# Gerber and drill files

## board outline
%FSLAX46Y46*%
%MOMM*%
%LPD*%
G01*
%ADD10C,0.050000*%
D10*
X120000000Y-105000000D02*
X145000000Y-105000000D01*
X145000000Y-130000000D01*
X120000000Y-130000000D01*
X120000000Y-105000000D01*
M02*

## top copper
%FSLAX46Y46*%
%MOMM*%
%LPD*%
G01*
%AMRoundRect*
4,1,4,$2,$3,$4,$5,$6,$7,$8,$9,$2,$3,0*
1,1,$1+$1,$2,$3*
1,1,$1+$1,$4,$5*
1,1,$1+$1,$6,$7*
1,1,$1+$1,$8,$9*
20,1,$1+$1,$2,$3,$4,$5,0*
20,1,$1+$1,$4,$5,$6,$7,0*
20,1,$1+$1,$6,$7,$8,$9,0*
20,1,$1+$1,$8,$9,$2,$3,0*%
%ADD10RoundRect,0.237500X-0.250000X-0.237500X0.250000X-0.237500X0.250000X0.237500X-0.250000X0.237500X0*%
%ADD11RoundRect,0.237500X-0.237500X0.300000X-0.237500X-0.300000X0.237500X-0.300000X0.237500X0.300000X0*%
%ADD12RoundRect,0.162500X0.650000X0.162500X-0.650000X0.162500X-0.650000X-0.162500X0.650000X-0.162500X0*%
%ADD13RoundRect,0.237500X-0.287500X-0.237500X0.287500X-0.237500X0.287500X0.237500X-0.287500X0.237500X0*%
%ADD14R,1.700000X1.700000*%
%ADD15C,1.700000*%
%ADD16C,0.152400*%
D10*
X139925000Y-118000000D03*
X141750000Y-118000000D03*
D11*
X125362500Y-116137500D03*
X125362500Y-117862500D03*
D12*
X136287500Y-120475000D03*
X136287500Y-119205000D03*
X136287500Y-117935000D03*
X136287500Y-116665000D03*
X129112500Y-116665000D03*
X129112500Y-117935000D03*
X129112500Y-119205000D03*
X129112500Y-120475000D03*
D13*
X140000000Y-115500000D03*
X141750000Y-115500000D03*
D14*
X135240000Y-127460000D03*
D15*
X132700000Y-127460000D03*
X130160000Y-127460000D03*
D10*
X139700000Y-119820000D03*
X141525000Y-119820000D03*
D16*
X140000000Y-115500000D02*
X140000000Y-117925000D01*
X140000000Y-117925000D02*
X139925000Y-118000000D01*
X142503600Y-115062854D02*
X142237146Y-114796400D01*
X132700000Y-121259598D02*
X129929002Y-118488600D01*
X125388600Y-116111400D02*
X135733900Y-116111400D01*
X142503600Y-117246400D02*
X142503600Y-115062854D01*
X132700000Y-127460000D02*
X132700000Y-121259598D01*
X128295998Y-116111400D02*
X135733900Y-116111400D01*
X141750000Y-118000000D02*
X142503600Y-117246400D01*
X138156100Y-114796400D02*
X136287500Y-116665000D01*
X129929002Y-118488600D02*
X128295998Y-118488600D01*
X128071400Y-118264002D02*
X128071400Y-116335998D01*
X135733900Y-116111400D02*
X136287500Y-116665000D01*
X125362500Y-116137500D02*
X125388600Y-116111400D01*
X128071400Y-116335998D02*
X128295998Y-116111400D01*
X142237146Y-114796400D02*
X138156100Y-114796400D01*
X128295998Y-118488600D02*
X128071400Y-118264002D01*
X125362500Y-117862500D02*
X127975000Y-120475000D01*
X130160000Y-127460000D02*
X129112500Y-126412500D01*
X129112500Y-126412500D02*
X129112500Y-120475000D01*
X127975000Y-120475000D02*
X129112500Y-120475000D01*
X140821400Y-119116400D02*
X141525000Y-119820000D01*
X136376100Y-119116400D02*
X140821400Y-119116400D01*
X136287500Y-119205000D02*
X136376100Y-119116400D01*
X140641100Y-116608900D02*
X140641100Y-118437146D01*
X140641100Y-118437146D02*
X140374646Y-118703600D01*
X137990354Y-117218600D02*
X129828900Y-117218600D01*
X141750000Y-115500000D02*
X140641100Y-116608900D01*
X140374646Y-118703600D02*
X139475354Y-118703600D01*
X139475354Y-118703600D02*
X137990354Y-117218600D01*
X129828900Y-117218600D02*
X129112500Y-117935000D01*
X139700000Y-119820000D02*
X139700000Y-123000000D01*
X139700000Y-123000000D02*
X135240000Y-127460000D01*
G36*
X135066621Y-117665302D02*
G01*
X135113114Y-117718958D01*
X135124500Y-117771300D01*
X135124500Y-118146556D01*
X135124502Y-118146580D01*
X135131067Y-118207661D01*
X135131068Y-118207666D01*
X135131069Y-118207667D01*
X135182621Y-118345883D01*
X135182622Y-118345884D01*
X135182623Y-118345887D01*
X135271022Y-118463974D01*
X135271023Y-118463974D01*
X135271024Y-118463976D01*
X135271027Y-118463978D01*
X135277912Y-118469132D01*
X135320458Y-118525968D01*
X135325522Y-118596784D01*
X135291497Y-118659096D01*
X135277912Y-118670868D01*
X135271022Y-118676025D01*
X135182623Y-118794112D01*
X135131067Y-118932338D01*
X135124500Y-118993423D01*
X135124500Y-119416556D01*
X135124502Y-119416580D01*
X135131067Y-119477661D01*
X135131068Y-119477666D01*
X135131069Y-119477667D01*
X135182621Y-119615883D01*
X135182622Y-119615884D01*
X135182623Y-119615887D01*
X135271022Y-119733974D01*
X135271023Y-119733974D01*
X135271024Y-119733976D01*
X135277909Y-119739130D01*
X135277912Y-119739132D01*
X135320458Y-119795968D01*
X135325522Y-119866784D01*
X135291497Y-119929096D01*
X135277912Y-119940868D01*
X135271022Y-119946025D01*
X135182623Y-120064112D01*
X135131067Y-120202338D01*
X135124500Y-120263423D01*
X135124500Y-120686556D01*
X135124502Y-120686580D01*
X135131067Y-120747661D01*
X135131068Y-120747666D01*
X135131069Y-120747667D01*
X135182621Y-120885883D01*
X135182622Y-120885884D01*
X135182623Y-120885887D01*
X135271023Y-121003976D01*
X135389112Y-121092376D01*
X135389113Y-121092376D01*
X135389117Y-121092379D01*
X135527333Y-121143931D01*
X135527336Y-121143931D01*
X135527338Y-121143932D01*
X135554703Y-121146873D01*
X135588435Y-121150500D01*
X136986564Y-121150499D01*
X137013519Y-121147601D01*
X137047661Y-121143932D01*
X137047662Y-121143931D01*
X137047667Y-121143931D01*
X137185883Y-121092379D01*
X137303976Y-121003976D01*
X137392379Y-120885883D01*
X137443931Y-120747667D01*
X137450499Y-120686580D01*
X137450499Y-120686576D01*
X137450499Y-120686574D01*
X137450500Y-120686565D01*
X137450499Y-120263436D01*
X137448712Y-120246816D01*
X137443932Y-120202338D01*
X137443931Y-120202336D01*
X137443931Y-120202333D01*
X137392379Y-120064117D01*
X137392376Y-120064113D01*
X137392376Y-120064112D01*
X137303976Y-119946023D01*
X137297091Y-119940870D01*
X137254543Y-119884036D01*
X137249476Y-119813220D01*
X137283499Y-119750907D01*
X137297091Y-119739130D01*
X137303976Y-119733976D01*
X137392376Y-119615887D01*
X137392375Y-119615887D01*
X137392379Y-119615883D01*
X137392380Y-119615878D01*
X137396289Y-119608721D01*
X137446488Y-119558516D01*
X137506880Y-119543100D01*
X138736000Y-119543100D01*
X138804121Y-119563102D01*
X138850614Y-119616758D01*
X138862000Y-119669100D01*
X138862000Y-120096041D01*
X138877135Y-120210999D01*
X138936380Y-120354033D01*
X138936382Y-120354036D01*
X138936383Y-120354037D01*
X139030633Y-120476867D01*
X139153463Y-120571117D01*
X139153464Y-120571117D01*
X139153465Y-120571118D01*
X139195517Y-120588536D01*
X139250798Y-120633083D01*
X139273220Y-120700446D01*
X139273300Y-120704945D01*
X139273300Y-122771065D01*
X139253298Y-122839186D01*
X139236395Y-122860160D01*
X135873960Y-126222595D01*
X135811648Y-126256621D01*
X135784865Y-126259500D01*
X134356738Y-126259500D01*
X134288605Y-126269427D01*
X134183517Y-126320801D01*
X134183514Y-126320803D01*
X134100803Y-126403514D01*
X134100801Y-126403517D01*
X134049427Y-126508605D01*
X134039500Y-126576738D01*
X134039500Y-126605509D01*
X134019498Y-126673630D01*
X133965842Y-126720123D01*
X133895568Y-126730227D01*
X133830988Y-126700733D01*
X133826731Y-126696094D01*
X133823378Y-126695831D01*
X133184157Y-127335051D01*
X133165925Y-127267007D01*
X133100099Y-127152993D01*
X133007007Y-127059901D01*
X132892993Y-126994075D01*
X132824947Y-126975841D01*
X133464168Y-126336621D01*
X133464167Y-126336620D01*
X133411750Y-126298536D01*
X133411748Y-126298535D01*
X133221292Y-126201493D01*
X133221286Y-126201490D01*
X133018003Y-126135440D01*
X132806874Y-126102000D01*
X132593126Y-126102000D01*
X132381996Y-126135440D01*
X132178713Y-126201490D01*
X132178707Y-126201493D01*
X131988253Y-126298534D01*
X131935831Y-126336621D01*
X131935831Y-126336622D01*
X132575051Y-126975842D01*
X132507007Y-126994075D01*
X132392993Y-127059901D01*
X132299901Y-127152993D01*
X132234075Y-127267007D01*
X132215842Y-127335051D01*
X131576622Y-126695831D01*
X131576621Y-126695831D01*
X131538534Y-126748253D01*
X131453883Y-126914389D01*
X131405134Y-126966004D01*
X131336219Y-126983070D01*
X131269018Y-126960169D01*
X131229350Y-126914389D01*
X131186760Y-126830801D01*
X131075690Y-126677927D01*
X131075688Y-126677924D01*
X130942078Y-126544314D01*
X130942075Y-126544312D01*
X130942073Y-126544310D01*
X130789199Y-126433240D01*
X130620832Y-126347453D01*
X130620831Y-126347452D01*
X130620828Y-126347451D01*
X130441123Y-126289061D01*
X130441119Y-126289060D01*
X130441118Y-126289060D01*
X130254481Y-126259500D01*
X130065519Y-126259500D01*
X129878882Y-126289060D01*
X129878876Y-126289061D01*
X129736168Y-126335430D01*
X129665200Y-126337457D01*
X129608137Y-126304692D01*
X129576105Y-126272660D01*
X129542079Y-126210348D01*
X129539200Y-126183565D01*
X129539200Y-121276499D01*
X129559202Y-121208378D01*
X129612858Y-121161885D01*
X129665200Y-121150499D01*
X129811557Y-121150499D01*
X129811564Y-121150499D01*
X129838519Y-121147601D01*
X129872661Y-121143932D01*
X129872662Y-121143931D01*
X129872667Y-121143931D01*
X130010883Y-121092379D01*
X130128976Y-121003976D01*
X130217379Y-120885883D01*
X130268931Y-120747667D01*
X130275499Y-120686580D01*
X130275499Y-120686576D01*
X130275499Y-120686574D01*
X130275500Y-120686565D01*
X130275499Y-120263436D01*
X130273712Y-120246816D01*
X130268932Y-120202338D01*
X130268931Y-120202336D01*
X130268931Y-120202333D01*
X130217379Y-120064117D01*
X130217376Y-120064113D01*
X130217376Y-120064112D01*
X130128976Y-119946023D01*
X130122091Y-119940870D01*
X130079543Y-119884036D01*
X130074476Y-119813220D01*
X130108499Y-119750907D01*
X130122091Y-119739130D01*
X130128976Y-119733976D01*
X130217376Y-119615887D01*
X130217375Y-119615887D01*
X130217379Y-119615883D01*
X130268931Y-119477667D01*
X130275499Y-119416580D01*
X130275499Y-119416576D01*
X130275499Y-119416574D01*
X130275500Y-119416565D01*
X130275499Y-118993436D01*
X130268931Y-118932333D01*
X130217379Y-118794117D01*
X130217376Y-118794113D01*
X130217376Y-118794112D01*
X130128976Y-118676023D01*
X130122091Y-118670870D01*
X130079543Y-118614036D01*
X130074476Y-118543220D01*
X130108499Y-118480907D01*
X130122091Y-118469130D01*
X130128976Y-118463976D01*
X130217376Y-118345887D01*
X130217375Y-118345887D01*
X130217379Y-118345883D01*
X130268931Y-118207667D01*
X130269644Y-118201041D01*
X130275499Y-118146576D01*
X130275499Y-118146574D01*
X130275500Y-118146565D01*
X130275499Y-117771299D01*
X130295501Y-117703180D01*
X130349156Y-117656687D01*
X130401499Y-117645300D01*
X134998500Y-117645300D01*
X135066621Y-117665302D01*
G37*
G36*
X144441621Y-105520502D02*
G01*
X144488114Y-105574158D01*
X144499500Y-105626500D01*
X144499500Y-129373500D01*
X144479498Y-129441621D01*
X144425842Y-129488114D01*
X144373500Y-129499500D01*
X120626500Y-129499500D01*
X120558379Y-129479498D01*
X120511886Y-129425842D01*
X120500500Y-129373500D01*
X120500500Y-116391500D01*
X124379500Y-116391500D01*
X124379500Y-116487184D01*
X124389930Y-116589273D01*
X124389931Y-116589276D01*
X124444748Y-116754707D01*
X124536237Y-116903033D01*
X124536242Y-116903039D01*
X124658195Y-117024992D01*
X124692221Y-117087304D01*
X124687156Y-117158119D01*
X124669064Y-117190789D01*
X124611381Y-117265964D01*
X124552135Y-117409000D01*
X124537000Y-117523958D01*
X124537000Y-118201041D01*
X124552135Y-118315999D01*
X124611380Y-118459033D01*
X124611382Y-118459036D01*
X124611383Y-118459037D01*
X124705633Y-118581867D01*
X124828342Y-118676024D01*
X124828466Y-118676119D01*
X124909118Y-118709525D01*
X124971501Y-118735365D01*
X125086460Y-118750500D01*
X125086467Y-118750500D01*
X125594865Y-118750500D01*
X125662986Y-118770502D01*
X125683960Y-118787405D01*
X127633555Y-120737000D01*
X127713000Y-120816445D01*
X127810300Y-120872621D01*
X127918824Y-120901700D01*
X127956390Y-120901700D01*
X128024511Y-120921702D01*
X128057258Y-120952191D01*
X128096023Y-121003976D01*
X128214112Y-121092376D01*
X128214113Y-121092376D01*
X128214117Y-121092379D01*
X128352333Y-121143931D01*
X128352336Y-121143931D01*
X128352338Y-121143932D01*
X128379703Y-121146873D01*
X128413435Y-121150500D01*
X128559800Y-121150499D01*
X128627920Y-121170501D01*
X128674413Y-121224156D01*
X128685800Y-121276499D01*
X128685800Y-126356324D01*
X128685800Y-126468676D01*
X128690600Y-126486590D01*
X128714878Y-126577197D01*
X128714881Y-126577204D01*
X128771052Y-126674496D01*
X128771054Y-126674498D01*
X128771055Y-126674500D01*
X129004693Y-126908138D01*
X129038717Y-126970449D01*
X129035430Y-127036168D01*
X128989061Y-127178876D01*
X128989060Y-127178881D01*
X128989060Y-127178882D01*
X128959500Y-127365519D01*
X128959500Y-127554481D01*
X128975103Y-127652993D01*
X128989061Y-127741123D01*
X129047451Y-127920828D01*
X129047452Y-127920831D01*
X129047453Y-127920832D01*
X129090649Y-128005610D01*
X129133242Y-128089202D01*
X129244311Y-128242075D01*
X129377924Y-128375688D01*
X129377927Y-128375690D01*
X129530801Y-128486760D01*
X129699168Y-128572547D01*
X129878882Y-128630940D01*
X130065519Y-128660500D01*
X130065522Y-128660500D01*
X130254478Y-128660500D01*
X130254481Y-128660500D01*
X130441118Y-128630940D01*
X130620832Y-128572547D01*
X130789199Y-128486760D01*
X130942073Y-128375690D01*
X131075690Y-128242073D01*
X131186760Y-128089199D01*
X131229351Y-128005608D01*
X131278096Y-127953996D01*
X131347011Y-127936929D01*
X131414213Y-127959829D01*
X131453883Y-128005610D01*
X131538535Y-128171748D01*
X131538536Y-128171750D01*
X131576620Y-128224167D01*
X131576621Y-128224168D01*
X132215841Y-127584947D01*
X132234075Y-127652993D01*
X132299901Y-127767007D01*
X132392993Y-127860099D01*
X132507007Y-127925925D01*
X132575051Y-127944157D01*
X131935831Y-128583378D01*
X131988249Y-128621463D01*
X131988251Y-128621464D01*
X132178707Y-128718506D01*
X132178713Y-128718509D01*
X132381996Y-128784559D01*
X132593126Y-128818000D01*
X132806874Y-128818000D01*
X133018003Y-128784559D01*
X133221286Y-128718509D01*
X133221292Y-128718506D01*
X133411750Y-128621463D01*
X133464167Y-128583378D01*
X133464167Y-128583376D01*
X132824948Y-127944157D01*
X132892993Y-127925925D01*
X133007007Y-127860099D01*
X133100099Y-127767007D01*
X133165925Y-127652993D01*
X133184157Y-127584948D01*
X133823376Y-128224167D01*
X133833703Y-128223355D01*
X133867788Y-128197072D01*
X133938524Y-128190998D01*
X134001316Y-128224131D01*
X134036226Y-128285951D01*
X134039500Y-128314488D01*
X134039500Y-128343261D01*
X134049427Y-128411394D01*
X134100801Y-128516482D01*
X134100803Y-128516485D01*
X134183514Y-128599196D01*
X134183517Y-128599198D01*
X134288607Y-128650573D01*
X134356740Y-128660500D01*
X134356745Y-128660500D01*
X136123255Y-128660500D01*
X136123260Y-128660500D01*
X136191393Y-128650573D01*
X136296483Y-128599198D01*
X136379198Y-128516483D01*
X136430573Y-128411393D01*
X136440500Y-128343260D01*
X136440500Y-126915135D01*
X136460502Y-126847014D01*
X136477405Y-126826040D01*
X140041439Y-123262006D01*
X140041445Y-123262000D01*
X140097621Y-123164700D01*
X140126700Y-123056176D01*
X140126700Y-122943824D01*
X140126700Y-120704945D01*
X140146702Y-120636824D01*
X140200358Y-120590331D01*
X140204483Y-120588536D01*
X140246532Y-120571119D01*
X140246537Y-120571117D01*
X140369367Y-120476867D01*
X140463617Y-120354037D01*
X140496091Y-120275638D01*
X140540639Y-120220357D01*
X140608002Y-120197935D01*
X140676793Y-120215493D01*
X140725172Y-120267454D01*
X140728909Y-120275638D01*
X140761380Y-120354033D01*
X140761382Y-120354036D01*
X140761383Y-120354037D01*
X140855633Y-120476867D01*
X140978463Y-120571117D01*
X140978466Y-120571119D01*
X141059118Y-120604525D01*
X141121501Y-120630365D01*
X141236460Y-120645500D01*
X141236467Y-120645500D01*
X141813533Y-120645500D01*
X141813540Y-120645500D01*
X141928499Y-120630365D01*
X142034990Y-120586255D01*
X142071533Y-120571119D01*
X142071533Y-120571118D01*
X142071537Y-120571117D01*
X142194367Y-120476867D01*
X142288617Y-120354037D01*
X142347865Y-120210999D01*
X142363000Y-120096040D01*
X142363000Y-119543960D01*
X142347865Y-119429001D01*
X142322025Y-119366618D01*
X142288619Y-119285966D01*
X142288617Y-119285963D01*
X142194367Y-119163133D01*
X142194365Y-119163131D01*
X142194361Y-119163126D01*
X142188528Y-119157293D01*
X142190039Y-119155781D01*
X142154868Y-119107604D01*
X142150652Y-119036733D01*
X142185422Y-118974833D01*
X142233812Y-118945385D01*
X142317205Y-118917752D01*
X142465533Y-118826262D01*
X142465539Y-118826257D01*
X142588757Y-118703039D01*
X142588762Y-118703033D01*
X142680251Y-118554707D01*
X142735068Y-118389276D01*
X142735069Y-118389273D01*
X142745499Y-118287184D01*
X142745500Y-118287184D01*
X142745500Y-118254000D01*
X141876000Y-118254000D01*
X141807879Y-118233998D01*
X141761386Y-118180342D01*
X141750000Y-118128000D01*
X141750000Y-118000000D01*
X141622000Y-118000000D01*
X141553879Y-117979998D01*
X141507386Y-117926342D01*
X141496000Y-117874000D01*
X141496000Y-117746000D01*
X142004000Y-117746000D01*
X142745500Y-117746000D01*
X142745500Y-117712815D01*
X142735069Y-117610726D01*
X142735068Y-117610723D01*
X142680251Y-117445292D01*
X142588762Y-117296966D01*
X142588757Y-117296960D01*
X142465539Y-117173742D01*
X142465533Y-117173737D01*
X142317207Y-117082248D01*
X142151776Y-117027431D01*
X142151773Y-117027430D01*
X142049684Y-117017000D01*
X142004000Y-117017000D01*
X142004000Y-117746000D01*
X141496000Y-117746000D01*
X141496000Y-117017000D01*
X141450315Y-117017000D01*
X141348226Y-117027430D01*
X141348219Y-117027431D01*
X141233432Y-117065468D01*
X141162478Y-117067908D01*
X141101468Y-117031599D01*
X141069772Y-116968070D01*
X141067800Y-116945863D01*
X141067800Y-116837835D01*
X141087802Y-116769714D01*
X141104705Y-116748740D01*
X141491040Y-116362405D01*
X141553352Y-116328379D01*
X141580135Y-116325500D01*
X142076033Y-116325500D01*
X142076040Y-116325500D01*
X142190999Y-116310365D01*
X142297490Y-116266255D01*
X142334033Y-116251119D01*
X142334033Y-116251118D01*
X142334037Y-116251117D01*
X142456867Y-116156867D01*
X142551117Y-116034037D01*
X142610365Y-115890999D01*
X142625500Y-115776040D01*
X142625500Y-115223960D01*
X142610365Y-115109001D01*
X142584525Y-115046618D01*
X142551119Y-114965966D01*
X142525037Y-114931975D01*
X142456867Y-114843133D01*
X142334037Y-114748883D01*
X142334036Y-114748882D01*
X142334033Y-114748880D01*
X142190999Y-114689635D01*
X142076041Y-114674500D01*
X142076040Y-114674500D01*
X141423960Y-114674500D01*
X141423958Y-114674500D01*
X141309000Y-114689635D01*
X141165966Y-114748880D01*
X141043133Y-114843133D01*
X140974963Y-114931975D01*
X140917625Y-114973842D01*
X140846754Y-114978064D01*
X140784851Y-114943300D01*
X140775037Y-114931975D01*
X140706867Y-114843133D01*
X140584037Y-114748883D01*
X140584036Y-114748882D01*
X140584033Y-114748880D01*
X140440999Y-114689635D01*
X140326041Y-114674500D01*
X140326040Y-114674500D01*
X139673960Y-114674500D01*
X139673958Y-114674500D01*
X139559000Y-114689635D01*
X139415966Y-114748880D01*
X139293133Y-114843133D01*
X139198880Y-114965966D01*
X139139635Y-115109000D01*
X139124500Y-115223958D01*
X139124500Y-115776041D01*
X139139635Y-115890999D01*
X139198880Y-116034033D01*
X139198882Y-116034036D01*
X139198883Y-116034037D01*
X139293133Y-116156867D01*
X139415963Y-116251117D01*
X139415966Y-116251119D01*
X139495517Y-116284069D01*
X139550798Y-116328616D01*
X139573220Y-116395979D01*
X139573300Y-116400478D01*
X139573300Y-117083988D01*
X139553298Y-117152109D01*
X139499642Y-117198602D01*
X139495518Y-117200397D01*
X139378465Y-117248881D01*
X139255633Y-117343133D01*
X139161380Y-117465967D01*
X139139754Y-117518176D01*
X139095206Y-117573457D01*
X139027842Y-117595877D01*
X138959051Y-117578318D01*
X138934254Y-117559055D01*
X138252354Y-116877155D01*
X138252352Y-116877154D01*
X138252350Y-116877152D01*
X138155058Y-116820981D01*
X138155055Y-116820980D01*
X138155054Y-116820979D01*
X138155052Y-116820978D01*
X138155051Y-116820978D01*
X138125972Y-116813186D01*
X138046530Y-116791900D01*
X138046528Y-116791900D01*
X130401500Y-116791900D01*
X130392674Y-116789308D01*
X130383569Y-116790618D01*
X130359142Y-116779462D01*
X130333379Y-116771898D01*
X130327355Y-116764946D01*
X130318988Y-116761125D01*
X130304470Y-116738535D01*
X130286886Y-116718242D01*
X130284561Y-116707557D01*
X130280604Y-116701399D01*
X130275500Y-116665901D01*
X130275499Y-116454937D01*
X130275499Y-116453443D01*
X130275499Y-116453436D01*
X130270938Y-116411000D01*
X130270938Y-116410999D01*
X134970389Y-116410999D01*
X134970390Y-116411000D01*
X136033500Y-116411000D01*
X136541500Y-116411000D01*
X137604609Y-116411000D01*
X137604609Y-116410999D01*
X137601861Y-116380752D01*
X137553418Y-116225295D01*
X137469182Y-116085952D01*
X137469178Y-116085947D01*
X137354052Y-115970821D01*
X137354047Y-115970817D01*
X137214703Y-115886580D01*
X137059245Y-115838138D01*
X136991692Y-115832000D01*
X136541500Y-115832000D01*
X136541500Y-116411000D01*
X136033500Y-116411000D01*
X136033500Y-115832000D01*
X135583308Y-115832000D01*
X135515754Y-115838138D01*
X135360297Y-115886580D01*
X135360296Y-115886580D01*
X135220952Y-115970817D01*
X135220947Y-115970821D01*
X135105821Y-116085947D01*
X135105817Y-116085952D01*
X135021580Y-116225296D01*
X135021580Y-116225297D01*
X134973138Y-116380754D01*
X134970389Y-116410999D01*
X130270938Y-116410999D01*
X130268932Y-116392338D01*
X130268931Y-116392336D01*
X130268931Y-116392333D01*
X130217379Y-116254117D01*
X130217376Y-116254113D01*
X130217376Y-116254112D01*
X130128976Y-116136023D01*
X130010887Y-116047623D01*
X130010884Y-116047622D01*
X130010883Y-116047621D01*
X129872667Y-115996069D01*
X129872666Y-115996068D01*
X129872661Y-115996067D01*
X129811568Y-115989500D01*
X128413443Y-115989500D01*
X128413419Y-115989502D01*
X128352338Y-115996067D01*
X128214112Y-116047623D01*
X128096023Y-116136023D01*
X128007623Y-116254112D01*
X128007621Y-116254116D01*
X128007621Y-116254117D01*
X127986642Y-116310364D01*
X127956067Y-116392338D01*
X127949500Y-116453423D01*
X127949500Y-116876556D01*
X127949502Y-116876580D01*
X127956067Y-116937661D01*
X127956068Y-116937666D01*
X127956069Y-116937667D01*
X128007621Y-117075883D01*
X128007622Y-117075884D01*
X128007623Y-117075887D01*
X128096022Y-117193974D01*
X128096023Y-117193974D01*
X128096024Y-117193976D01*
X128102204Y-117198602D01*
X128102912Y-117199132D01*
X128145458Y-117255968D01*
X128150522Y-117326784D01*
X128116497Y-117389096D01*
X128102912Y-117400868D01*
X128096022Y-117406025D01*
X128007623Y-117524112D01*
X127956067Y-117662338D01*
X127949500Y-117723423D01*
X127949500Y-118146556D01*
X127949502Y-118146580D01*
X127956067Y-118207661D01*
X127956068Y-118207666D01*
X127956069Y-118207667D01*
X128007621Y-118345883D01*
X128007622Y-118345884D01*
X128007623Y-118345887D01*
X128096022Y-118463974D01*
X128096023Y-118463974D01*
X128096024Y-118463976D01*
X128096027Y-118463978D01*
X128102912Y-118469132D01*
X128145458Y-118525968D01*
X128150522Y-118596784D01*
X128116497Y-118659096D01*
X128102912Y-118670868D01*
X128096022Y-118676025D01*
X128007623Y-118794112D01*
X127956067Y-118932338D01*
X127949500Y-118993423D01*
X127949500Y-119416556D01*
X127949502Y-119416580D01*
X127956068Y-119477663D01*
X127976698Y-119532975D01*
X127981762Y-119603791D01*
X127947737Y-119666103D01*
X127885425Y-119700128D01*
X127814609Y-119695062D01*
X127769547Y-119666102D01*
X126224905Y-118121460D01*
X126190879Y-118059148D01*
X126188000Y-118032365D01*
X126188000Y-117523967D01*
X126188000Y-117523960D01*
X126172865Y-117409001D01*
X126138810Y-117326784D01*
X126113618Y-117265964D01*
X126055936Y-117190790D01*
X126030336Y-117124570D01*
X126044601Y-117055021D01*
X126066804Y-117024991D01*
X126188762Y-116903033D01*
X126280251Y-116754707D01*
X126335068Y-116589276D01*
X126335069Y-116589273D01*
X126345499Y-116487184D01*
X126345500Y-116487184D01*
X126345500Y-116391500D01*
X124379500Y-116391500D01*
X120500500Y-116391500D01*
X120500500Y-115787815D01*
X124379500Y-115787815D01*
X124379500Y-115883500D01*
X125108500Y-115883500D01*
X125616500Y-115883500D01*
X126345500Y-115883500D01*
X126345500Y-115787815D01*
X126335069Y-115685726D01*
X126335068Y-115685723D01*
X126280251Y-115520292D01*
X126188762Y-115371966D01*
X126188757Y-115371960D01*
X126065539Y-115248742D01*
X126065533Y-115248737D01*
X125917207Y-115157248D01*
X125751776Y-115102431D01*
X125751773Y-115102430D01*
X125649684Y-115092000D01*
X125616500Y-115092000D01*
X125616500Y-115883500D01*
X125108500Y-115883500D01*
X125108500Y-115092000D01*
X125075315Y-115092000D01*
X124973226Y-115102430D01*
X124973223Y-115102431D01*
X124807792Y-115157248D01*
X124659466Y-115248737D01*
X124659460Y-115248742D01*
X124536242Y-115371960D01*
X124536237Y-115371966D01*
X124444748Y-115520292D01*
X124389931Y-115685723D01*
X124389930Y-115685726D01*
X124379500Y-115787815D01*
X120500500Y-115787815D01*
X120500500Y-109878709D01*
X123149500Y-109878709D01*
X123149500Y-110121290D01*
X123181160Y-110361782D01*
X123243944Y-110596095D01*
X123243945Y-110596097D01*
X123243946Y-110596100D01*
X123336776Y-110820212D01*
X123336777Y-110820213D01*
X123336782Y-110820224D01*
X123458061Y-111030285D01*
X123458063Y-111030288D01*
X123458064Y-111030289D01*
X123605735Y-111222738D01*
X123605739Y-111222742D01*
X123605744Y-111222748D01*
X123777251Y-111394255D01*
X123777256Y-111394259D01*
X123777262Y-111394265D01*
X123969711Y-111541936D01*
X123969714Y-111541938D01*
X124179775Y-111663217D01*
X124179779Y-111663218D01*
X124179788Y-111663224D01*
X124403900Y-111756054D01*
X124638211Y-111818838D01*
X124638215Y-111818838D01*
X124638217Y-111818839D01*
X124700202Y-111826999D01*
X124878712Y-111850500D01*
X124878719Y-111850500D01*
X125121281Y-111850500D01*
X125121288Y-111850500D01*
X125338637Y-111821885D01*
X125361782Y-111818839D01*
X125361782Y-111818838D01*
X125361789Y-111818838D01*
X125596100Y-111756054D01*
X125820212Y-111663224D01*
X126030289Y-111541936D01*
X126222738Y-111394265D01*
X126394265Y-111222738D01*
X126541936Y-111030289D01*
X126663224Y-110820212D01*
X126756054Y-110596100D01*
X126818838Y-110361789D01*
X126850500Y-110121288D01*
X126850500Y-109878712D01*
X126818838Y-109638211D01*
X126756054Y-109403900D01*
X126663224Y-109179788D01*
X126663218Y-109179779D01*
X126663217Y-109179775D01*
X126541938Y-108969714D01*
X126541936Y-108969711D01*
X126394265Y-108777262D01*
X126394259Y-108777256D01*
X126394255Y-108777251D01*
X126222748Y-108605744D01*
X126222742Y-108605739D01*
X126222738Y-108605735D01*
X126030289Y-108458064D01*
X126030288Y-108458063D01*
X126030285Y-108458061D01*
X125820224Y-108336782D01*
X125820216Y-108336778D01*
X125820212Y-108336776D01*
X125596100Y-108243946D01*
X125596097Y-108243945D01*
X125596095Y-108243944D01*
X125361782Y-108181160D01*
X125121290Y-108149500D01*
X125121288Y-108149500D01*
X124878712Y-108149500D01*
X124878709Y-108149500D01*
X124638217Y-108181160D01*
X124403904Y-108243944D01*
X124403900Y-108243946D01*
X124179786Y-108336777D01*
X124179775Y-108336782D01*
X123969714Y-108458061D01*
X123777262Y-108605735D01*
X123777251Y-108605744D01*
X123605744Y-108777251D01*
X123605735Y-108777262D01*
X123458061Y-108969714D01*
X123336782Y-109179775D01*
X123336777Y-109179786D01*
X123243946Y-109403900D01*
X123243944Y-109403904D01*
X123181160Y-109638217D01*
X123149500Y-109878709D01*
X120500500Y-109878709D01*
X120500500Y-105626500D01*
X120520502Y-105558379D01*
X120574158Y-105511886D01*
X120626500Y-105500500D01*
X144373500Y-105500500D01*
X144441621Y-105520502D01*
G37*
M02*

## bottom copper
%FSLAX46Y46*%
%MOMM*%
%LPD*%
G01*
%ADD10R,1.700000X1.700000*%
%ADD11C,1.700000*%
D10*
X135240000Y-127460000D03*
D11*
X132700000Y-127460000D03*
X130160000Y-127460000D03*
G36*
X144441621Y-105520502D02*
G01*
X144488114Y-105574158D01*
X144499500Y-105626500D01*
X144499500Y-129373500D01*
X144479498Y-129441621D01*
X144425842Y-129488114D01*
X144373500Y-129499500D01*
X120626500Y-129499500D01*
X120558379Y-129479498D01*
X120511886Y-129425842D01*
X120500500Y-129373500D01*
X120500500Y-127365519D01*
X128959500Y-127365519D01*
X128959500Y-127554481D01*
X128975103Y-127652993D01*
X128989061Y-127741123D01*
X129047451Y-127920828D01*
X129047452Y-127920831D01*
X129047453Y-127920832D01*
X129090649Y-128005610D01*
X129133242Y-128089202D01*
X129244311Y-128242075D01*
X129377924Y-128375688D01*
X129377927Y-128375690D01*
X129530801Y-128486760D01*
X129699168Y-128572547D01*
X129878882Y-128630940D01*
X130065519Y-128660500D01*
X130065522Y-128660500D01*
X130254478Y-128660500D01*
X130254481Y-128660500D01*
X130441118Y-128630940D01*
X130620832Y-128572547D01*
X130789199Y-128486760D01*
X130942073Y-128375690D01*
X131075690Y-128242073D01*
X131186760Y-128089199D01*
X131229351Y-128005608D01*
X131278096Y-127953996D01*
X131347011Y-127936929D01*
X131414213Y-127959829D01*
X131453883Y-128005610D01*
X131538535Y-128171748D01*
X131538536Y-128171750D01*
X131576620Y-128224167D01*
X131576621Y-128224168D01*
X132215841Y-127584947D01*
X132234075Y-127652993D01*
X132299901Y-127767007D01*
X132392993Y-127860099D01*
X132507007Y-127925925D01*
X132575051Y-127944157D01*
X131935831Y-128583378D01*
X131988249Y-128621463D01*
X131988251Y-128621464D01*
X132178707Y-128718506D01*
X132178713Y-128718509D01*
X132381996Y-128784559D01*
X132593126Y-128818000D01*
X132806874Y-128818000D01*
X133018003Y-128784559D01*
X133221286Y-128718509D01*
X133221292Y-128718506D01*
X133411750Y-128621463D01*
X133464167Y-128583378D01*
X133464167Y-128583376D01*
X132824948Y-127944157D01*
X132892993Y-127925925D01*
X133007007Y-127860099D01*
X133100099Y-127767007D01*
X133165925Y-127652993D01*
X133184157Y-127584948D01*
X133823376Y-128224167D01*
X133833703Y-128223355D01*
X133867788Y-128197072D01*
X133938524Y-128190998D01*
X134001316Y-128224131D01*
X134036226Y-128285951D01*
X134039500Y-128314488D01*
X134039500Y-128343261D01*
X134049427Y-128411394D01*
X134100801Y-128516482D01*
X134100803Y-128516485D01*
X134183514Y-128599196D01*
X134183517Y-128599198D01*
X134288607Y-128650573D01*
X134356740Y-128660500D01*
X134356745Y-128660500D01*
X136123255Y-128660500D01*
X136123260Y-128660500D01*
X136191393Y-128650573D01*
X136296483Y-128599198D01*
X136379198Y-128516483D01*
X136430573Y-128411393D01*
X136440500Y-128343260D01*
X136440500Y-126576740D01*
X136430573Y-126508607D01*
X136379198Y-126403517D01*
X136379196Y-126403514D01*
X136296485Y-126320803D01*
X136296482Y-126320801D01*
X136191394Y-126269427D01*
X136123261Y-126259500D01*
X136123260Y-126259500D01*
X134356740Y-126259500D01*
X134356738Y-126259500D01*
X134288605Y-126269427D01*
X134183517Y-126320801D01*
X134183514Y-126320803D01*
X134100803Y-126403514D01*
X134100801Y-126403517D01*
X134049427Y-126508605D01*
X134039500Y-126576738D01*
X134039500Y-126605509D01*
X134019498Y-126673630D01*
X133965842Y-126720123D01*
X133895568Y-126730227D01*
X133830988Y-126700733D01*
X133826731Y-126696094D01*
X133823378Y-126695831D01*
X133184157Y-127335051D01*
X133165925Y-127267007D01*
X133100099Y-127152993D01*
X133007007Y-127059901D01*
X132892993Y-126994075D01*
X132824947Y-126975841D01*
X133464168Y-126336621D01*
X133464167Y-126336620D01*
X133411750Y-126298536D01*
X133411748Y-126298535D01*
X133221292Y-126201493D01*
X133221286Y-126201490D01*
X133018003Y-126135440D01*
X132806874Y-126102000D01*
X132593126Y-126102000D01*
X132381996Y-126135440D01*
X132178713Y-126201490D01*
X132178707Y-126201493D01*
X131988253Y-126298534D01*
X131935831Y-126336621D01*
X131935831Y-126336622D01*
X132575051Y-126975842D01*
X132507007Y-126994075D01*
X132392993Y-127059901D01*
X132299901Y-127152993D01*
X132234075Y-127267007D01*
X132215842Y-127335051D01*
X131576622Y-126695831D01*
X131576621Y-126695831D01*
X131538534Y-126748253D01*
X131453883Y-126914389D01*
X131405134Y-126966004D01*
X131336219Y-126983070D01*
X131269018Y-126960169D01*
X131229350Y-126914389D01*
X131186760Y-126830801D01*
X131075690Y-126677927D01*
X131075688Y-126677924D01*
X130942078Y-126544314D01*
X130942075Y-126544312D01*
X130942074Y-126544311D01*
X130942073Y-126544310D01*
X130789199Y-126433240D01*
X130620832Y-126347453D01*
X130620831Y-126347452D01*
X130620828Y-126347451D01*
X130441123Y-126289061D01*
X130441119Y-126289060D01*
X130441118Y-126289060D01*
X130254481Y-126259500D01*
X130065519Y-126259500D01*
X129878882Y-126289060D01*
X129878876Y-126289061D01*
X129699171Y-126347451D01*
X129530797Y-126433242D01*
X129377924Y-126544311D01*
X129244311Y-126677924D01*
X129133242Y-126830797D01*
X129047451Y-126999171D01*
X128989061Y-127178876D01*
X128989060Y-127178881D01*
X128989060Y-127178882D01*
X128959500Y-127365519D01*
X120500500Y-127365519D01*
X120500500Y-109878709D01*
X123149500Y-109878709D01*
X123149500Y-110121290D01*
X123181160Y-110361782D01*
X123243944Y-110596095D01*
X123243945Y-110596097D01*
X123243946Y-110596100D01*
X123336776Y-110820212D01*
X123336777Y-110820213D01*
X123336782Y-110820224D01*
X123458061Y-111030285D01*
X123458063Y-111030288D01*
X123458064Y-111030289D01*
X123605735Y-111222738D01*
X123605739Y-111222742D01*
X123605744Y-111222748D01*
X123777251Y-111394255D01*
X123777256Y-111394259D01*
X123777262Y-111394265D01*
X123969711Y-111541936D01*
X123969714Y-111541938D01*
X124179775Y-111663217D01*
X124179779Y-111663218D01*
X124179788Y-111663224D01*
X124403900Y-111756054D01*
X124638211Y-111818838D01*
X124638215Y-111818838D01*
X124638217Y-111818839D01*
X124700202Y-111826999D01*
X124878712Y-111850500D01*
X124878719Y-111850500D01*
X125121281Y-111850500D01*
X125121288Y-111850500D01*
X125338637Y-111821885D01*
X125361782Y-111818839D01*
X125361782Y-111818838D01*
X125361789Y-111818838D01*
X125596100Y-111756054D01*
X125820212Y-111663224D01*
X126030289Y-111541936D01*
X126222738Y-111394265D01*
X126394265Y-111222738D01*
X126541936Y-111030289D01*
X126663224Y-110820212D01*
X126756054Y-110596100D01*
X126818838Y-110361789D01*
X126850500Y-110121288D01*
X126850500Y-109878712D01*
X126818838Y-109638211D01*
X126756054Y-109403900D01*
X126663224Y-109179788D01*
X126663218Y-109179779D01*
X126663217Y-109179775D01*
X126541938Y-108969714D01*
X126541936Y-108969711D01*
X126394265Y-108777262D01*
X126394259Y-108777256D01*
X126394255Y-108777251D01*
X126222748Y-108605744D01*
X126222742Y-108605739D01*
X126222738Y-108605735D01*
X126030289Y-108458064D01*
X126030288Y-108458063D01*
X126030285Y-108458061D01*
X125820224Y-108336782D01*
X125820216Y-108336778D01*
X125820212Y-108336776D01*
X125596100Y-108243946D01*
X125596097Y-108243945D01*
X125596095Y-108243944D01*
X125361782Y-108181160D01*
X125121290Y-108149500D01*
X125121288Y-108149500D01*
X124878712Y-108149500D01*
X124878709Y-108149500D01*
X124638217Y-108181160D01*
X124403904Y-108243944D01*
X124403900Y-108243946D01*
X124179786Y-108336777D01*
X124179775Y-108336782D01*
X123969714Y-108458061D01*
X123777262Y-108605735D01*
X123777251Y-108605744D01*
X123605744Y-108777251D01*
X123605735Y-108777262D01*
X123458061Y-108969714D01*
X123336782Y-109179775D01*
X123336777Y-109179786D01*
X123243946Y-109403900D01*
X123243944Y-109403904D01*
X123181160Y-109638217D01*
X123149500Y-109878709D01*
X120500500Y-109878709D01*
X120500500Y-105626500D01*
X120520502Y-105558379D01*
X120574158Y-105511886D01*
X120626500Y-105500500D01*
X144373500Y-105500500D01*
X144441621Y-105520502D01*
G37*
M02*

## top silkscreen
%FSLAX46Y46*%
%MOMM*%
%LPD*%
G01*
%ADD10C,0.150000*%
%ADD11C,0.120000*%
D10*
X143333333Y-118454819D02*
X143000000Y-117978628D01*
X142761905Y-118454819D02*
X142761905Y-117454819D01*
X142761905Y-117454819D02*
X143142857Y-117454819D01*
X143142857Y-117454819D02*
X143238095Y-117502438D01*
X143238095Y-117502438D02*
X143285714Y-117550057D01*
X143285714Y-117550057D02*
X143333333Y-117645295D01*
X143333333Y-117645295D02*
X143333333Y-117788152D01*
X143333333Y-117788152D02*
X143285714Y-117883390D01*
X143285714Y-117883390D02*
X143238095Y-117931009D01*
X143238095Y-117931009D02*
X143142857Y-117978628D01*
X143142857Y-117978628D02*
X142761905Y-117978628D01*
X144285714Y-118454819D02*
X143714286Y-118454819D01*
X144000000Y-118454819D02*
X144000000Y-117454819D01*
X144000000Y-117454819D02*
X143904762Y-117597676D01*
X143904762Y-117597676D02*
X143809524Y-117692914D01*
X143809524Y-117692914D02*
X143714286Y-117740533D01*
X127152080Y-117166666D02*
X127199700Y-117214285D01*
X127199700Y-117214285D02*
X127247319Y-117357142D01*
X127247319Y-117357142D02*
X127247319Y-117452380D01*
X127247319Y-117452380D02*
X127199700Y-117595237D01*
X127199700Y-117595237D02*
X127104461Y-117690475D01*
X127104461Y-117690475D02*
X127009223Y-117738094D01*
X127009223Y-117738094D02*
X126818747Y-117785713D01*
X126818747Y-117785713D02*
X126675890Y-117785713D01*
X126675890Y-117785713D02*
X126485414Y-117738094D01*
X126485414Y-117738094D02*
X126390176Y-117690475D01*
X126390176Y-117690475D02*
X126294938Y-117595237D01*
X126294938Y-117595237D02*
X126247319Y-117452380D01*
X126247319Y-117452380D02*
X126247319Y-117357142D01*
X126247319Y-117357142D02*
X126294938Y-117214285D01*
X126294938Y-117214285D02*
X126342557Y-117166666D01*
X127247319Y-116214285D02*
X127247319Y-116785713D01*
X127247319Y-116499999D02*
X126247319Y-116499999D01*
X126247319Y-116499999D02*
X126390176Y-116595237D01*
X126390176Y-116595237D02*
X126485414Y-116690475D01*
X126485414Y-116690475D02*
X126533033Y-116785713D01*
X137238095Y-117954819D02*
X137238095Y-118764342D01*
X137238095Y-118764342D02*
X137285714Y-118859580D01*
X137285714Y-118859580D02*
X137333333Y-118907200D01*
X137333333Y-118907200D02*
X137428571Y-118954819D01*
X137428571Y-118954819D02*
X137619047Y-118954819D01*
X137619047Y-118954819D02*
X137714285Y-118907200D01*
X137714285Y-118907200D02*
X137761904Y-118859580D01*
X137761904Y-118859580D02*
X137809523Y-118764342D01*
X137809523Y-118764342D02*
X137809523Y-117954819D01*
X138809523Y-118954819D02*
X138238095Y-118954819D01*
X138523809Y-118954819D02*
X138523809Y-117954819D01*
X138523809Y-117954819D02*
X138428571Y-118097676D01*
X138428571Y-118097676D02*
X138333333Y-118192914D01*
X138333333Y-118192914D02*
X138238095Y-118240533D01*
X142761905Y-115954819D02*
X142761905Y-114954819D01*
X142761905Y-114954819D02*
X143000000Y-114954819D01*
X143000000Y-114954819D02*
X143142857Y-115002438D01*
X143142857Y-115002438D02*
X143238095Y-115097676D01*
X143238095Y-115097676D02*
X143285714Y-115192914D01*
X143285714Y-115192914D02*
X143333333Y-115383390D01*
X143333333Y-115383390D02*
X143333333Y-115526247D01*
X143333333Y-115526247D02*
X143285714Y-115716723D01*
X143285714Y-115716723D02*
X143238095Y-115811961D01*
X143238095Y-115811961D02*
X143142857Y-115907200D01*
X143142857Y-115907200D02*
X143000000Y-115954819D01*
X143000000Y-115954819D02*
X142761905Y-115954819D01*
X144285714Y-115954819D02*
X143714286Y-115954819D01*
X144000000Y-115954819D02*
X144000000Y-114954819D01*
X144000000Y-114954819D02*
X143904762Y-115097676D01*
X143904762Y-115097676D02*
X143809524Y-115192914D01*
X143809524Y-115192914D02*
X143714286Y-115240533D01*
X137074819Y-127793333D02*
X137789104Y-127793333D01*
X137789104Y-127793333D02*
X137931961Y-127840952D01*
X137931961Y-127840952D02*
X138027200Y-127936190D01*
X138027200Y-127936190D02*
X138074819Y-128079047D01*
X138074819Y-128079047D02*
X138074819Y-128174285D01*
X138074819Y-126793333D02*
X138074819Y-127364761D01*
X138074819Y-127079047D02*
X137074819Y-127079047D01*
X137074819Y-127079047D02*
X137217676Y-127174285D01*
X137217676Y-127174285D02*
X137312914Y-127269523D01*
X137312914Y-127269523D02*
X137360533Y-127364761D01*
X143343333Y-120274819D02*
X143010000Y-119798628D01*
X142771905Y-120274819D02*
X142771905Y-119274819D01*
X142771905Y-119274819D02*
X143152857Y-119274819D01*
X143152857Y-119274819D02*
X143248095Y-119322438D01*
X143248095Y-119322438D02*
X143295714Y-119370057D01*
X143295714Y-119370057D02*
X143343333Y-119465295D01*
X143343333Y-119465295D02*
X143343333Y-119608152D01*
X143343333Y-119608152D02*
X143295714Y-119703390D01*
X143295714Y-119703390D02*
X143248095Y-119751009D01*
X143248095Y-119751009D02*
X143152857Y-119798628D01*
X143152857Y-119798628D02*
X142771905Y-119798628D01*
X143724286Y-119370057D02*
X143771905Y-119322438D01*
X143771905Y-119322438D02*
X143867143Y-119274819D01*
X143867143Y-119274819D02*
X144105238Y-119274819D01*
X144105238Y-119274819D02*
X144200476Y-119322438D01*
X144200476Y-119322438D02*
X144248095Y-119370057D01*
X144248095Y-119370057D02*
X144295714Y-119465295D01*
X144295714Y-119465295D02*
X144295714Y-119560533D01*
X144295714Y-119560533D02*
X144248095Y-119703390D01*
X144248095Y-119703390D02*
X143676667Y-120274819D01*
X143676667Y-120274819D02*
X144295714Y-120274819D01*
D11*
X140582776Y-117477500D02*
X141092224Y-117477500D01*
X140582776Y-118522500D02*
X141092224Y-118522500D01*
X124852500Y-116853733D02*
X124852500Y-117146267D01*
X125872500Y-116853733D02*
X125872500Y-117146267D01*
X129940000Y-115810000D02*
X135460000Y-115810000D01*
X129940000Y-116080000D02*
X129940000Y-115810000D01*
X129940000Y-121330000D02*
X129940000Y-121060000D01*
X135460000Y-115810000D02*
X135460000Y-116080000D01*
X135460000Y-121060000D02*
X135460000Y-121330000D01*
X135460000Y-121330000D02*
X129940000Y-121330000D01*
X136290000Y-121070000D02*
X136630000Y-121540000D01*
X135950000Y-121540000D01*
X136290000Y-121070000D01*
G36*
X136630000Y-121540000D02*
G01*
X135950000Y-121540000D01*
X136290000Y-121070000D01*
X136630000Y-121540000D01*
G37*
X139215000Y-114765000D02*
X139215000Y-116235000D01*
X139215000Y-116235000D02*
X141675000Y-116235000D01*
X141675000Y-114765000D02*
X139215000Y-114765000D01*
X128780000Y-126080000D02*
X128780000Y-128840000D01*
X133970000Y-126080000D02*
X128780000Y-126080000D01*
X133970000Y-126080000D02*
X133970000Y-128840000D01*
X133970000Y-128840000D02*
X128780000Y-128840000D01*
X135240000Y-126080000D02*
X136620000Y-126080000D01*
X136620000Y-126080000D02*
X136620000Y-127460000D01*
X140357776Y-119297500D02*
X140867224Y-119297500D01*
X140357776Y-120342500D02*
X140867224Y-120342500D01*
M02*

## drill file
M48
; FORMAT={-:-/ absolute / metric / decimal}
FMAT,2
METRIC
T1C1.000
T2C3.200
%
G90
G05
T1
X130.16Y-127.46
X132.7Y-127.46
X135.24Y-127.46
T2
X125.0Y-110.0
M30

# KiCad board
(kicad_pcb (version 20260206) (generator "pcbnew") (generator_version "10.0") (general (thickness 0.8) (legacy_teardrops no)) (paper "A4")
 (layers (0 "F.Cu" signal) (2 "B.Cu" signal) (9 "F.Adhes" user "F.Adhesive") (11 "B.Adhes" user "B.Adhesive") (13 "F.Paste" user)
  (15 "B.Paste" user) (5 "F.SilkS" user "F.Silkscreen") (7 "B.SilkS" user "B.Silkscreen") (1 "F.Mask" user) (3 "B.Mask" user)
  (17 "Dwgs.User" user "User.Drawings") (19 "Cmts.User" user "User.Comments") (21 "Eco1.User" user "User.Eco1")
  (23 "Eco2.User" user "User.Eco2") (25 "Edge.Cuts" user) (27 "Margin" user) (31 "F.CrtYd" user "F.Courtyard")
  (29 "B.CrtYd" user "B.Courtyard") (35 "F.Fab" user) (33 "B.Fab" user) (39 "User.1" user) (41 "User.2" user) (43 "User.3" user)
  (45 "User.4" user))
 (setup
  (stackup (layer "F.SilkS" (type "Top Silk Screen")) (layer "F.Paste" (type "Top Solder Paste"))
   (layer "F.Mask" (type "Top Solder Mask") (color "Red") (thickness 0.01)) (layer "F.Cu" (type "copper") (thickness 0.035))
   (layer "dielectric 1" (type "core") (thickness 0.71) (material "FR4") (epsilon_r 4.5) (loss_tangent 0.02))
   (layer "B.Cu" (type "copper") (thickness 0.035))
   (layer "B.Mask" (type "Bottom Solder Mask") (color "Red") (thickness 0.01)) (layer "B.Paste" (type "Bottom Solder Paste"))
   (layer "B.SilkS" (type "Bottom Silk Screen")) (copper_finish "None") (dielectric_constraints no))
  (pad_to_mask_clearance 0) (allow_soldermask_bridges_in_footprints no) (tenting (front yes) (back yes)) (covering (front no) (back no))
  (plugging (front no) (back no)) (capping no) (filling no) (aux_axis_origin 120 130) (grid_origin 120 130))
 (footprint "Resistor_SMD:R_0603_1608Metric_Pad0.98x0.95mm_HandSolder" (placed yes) (layer "F.Cu") (at 140.8375 118)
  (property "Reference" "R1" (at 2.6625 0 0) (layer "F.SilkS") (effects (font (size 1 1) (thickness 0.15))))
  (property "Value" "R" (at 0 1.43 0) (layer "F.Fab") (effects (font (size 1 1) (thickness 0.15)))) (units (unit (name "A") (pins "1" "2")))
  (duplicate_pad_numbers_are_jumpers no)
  (fp_line (start -0.254724 -0.5225) (end 0.254724 -0.5225) (stroke (width 0.12) (type solid)) (layer "F.SilkS"))
  (fp_line (start -0.254724 0.5225) (end 0.254724 0.5225) (stroke (width 0.12) (type solid)) (layer "F.SilkS"))
  (pad "1" smd roundrect (at -0.9125 0) (size 0.975 0.95) (layers "F.Cu" "F.Mask" "F.Paste") (roundrect_rratio 0.25) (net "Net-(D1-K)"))
  (pad "2" smd roundrect (at 0.9125 0) (size 0.975 0.95) (layers "F.Cu" "F.Mask" "F.Paste") (roundrect_rratio 0.25) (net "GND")))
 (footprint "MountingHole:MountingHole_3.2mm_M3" (layer "F.Cu") (at 125 110)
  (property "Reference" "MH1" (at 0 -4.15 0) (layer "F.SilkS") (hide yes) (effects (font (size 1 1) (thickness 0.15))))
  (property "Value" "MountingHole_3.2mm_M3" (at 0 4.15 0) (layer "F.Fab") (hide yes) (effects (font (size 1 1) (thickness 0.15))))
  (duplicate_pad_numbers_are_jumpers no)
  (pad "" np_thru_hole circle (at 0 0) (size 3.2 3.2) (drill 3.2) (layers "*.Cu" "*.Mask")))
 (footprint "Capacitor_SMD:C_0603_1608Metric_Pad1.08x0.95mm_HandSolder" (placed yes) (layer "F.Cu") (at 125.3625 117 -90)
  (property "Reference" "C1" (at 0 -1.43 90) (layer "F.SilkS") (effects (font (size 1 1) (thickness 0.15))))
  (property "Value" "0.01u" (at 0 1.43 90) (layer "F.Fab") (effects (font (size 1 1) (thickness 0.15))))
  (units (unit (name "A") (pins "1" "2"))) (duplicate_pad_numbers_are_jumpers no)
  (fp_line (start -0.146267 0.51) (end 0.146267 0.51) (stroke (width 0.12) (type solid)) (layer "F.SilkS"))
  (fp_line (start -0.146267 -0.51) (end 0.146267 -0.51) (stroke (width 0.12) (type solid)) (layer "F.SilkS"))
  (pad "1" smd roundrect (at -0.8625 0 270) (size 1.075 0.95) (layers "F.Cu" "F.Mask" "F.Paste") (roundrect_rratio 0.25) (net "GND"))
  (pad "2" smd roundrect (at 0.8625 0 270) (size 1.075 0.95) (layers "F.Cu" "F.Mask" "F.Paste") (roundrect_rratio 0.25) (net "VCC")))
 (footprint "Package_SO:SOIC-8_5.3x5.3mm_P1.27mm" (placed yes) (layer "F.Cu") (at 132.7 118.57 180)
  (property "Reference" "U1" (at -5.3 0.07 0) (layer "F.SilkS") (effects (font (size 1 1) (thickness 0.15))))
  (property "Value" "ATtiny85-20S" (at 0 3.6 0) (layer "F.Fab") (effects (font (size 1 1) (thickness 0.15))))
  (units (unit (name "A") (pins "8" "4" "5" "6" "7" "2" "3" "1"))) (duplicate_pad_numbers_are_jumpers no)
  (fp_line (start 2.76 2.76) (end -2.76 2.76) (stroke (width 0.12) (type solid)) (layer "F.SilkS"))
  (fp_line (start 2.76 2.49) (end 2.76 2.76) (stroke (width 0.12) (type solid)) (layer "F.SilkS"))
  (fp_line (start 2.76 -2.76) (end 2.76 -2.49) (stroke (width 0.12) (type solid)) (layer "F.SilkS"))
  (fp_line (start -2.76 2.76) (end -2.76 2.49) (stroke (width 0.12) (type solid)) (layer "F.SilkS"))
  (fp_line (start -2.76 -2.49) (end -2.76 -2.76) (stroke (width 0.12) (type solid)) (layer "F.SilkS"))
  (fp_line (start -2.76 -2.76) (end 2.76 -2.76) (stroke (width 0.12) (type solid)) (layer "F.SilkS"))
  (fp_poly (pts (xy -3.59 -2.5) (xy -3.93 -2.97) (xy -3.25 -2.97)) (stroke (width 0.12) (type solid)) (fill yes) (layer "F.SilkS"))
  (pad "1" smd roundrect (at -3.5875 -1.905 180) (size 1.625 0.65) (layers "F.Cu" "F.Mask" "F.Paste") (roundrect_rratio 0.25)
   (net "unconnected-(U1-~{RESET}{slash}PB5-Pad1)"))
  (pad "2" smd roundrect (at -3.5875 -0.635 180) (size 1.625 0.65) (layers "F.Cu" "F.Mask" "F.Paste") (roundrect_rratio 0.25) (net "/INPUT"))
  (pad "3" smd roundrect (at -3.5875 0.635 180) (size 1.625 0.65) (layers "F.Cu" "F.Mask" "F.Paste") (roundrect_rratio 0.25)
   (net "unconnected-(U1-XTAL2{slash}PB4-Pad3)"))
  (pad "4" smd roundrect (at -3.5875 1.905 180) (size 1.625 0.65) (layers "F.Cu" "F.Mask" "F.Paste") (roundrect_rratio 0.25) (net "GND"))
  (pad "5" smd roundrect (at 3.5875 1.905 180) (size 1.625 0.65) (layers "F.Cu" "F.Mask" "F.Paste") (roundrect_rratio 0.25)
   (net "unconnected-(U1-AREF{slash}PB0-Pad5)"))
  (pad "6" smd roundrect (at 3.5875 0.635 180) (size 1.625 0.65) (layers "F.Cu" "F.Mask" "F.Paste") (roundrect_rratio 0.25)
   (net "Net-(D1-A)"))
  (pad "7" smd roundrect (at 3.5875 -0.635 180) (size 1.625 0.65) (layers "F.Cu" "F.Mask" "F.Paste") (roundrect_rratio 0.25)
   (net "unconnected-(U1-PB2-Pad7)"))
  (pad "8" smd roundrect (at 3.5875 -1.905 180) (size 1.625 0.65) (layers "F.Cu" "F.Mask" "F.Paste") (roundrect_rratio 0.25) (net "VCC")))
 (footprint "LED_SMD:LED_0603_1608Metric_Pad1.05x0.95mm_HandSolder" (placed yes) (layer "F.Cu") (at 140.875 115.5)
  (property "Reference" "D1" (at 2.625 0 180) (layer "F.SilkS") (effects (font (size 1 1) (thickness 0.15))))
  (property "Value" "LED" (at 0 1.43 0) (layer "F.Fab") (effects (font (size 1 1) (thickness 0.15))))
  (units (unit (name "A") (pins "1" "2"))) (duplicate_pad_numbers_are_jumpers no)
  (fp_line (start -1.66 -0.735) (end -1.66 0.735) (stroke (width 0.12) (type solid)) (layer "F.SilkS"))
  (fp_line (start -1.66 0.735) (end 0.8 0.735) (stroke (width 0.12) (type solid)) (layer "F.SilkS"))
  (fp_line (start 0.8 -0.735) (end -1.66 -0.735) (stroke (width 0.12) (type solid)) (layer "F.SilkS"))
  (pad "1" smd roundrect (at -0.875 0) (size 1.05 0.95) (layers "F.Cu" "F.Mask" "F.Paste") (roundrect_rratio 0.25) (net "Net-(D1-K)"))
  (pad "2" smd roundrect (at 0.875 0) (size 1.05 0.95) (layers "F.Cu" "F.Mask" "F.Paste") (roundrect_rratio 0.25) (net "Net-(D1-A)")))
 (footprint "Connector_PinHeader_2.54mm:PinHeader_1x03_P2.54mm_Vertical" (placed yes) (layer "F.Cu") (at 135.24 127.46 -90)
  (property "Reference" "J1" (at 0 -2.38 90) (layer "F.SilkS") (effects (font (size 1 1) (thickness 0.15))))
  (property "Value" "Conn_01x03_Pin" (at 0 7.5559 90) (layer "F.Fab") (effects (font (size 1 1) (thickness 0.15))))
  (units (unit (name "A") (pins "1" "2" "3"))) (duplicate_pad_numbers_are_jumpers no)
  (fp_line (start -1.38 6.46) (end 1.38 6.46) (stroke (width 0.12) (type solid)) (layer "F.SilkS"))
  (fp_line (start -1.38 1.27) (end -1.38 6.46) (stroke (width 0.12) (type solid)) (layer "F.SilkS"))
  (fp_line (start -1.38 1.27) (end 1.38 1.27) (stroke (width 0.12) (type solid)) (layer "F.SilkS"))
  (fp_line (start 1.38 1.27) (end 1.38 6.46) (stroke (width 0.12) (type solid)) (layer "F.SilkS"))
  (fp_line (start -1.38 0) (end -1.38 -1.38) (stroke (width 0.12) (type solid)) (layer "F.SilkS"))
  (fp_line (start -1.38 -1.38) (end 0 -1.38) (stroke (width 0.12) (type solid)) (layer "F.SilkS"))
  (pad "1" thru_hole rect (at 0 0 270) (size 1.7 1.7) (drill 1) (layers "*.Cu" "*.Mask") (remove_unused_layers no) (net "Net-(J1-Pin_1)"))
  (pad "2" thru_hole circle (at 0 2.54 270) (size 1.7 1.7) (drill 1) (layers "*.Cu" "*.Mask") (remove_unused_layers no) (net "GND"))
  (pad "3" thru_hole circle (at 0 5.08 270) (size 1.7 1.7) (drill 1) (layers "*.Cu" "*.Mask") (remove_unused_layers no) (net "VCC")))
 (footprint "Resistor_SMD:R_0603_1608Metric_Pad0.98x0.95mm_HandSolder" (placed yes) (layer "F.Cu") (at 140.6125 119.82)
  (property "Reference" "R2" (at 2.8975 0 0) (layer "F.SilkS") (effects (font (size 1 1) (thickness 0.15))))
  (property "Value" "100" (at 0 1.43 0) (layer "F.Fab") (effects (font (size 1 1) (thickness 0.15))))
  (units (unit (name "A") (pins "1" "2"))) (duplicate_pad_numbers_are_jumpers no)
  (fp_line (start -0.254724 -0.5225) (end 0.254724 -0.5225) (stroke (width 0.12) (type solid)) (layer "F.SilkS"))
  (fp_line (start -0.254724 0.5225) (end 0.254724 0.5225) (stroke (width 0.12) (type solid)) (layer "F.SilkS"))
  (pad "1" smd roundrect (at -0.9125 0) (size 0.975 0.95) (layers "F.Cu" "F.Mask" "F.Paste") (roundrect_rratio 0.25) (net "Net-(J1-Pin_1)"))
  (pad "2" smd roundrect (at 0.9125 0) (size 0.975 0.95) (layers "F.Cu" "F.Mask" "F.Paste") (roundrect_rratio 0.25) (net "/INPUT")))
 (gr_rect (start 120 105) (end 145 130) (stroke (width 0.05) (type solid)) (fill no) (layer "Edge.Cuts"))
 (segment (start 140 115.5) (end 140 117.925) (width 0.1524) (layer "F.Cu") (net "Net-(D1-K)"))
 (segment (start 140 117.925) (end 139.925 118) (width 0.1524) (layer "F.Cu") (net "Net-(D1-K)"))
 (segment (start 142.5036 115.062854) (end 142.237146 114.7964) (width 0.1524) (layer "F.Cu") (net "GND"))
 (segment (start 132.7 121.259598) (end 129.929002 118.4886) (width 0.1524) (layer "F.Cu") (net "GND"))
 (segment (start 125.3886 116.1114) (end 135.7339 116.1114) (width 0.1524) (layer "F.Cu") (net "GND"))
 (segment (start 142.5036 117.2464) (end 142.5036 115.062854) (width 0.1524) (layer "F.Cu") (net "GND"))
 (segment (start 132.7 127.46) (end 132.7 121.259598) (width 0.1524) (layer "F.Cu") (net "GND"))
 (segment (start 128.295998 116.1114) (end 135.7339 116.1114) (width 0.1524) (layer "F.Cu") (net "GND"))
 (segment (start 141.75 118) (end 142.5036 117.2464) (width 0.1524) (layer "F.Cu") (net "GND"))
 (segment (start 138.1561 114.7964) (end 136.2875 116.665) (width 0.1524) (layer "F.Cu") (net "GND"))
 (segment (start 129.929002 118.4886) (end 128.295998 118.4886) (width 0.1524) (layer "F.Cu") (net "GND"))
 (segment (start 128.0714 118.264002) (end 128.0714 116.335998) (width 0.1524) (layer "F.Cu") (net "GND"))
 (segment (start 135.7339 116.1114) (end 136.2875 116.665) (width 0.1524) (layer "F.Cu") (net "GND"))
 (segment (start 125.3625 116.1375) (end 125.3886 116.1114) (width 0.1524) (layer "F.Cu") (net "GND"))
 (segment (start 128.0714 116.335998) (end 128.295998 116.1114) (width 0.1524) (layer "F.Cu") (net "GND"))
 (segment (start 142.237146 114.7964) (end 138.1561 114.7964) (width 0.1524) (layer "F.Cu") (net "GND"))
 (segment (start 128.295998 118.4886) (end 128.0714 118.264002) (width 0.1524) (layer "F.Cu") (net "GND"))
 (segment (start 125.3625 117.8625) (end 127.975 120.475) (width 0.1524) (layer "F.Cu") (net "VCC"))
 (segment (start 130.16 127.46) (end 129.1125 126.4125) (width 0.1524) (layer "F.Cu") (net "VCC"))
 (segment (start 129.1125 126.4125) (end 129.1125 120.475) (width 0.1524) (layer "F.Cu") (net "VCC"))
 (segment (start 127.975 120.475) (end 129.1125 120.475) (width 0.1524) (layer "F.Cu") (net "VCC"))
 (segment (start 140.8214 119.1164) (end 141.525 119.82) (width 0.1524) (layer "F.Cu") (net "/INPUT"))
 (segment (start 136.3761 119.1164) (end 140.8214 119.1164) (width 0.1524) (layer "F.Cu") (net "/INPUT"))
 (segment (start 136.2875 119.205) (end 136.3761 119.1164) (width 0.1524) (layer "F.Cu") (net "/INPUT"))
 (segment (start 140.6411 116.6089) (end 140.6411 118.437146) (width 0.1524) (layer "F.Cu") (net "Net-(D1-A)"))
 (segment (start 140.6411 118.437146) (end 140.374646 118.7036) (width 0.1524) (layer "F.Cu") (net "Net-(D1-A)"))
 (segment (start 137.990354 117.2186) (end 129.8289 117.2186) (width 0.1524) (layer "F.Cu") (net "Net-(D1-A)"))
 (segment (start 141.75 115.5) (end 140.6411 116.6089) (width 0.1524) (layer "F.Cu") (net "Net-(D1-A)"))
 (segment (start 140.374646 118.7036) (end 139.475354 118.7036) (width 0.1524) (layer "F.Cu") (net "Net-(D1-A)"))
 (segment (start 139.475354 118.7036) (end 137.990354 117.2186) (width 0.1524) (layer "F.Cu") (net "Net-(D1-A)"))
 (segment (start 129.8289 117.2186) (end 129.1125 117.935) (width 0.1524) (layer "F.Cu") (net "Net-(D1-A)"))
 (segment (start 139.7 119.82) (end 139.7 123) (width 0.1524) (layer "F.Cu") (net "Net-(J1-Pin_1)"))
 (segment (start 139.7 123) (end 135.24 127.46) (width 0.1524) (layer "F.Cu") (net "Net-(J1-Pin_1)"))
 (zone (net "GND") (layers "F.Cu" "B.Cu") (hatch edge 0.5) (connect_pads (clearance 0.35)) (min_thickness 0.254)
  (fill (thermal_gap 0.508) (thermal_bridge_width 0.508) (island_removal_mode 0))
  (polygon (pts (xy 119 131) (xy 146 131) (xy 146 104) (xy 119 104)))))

